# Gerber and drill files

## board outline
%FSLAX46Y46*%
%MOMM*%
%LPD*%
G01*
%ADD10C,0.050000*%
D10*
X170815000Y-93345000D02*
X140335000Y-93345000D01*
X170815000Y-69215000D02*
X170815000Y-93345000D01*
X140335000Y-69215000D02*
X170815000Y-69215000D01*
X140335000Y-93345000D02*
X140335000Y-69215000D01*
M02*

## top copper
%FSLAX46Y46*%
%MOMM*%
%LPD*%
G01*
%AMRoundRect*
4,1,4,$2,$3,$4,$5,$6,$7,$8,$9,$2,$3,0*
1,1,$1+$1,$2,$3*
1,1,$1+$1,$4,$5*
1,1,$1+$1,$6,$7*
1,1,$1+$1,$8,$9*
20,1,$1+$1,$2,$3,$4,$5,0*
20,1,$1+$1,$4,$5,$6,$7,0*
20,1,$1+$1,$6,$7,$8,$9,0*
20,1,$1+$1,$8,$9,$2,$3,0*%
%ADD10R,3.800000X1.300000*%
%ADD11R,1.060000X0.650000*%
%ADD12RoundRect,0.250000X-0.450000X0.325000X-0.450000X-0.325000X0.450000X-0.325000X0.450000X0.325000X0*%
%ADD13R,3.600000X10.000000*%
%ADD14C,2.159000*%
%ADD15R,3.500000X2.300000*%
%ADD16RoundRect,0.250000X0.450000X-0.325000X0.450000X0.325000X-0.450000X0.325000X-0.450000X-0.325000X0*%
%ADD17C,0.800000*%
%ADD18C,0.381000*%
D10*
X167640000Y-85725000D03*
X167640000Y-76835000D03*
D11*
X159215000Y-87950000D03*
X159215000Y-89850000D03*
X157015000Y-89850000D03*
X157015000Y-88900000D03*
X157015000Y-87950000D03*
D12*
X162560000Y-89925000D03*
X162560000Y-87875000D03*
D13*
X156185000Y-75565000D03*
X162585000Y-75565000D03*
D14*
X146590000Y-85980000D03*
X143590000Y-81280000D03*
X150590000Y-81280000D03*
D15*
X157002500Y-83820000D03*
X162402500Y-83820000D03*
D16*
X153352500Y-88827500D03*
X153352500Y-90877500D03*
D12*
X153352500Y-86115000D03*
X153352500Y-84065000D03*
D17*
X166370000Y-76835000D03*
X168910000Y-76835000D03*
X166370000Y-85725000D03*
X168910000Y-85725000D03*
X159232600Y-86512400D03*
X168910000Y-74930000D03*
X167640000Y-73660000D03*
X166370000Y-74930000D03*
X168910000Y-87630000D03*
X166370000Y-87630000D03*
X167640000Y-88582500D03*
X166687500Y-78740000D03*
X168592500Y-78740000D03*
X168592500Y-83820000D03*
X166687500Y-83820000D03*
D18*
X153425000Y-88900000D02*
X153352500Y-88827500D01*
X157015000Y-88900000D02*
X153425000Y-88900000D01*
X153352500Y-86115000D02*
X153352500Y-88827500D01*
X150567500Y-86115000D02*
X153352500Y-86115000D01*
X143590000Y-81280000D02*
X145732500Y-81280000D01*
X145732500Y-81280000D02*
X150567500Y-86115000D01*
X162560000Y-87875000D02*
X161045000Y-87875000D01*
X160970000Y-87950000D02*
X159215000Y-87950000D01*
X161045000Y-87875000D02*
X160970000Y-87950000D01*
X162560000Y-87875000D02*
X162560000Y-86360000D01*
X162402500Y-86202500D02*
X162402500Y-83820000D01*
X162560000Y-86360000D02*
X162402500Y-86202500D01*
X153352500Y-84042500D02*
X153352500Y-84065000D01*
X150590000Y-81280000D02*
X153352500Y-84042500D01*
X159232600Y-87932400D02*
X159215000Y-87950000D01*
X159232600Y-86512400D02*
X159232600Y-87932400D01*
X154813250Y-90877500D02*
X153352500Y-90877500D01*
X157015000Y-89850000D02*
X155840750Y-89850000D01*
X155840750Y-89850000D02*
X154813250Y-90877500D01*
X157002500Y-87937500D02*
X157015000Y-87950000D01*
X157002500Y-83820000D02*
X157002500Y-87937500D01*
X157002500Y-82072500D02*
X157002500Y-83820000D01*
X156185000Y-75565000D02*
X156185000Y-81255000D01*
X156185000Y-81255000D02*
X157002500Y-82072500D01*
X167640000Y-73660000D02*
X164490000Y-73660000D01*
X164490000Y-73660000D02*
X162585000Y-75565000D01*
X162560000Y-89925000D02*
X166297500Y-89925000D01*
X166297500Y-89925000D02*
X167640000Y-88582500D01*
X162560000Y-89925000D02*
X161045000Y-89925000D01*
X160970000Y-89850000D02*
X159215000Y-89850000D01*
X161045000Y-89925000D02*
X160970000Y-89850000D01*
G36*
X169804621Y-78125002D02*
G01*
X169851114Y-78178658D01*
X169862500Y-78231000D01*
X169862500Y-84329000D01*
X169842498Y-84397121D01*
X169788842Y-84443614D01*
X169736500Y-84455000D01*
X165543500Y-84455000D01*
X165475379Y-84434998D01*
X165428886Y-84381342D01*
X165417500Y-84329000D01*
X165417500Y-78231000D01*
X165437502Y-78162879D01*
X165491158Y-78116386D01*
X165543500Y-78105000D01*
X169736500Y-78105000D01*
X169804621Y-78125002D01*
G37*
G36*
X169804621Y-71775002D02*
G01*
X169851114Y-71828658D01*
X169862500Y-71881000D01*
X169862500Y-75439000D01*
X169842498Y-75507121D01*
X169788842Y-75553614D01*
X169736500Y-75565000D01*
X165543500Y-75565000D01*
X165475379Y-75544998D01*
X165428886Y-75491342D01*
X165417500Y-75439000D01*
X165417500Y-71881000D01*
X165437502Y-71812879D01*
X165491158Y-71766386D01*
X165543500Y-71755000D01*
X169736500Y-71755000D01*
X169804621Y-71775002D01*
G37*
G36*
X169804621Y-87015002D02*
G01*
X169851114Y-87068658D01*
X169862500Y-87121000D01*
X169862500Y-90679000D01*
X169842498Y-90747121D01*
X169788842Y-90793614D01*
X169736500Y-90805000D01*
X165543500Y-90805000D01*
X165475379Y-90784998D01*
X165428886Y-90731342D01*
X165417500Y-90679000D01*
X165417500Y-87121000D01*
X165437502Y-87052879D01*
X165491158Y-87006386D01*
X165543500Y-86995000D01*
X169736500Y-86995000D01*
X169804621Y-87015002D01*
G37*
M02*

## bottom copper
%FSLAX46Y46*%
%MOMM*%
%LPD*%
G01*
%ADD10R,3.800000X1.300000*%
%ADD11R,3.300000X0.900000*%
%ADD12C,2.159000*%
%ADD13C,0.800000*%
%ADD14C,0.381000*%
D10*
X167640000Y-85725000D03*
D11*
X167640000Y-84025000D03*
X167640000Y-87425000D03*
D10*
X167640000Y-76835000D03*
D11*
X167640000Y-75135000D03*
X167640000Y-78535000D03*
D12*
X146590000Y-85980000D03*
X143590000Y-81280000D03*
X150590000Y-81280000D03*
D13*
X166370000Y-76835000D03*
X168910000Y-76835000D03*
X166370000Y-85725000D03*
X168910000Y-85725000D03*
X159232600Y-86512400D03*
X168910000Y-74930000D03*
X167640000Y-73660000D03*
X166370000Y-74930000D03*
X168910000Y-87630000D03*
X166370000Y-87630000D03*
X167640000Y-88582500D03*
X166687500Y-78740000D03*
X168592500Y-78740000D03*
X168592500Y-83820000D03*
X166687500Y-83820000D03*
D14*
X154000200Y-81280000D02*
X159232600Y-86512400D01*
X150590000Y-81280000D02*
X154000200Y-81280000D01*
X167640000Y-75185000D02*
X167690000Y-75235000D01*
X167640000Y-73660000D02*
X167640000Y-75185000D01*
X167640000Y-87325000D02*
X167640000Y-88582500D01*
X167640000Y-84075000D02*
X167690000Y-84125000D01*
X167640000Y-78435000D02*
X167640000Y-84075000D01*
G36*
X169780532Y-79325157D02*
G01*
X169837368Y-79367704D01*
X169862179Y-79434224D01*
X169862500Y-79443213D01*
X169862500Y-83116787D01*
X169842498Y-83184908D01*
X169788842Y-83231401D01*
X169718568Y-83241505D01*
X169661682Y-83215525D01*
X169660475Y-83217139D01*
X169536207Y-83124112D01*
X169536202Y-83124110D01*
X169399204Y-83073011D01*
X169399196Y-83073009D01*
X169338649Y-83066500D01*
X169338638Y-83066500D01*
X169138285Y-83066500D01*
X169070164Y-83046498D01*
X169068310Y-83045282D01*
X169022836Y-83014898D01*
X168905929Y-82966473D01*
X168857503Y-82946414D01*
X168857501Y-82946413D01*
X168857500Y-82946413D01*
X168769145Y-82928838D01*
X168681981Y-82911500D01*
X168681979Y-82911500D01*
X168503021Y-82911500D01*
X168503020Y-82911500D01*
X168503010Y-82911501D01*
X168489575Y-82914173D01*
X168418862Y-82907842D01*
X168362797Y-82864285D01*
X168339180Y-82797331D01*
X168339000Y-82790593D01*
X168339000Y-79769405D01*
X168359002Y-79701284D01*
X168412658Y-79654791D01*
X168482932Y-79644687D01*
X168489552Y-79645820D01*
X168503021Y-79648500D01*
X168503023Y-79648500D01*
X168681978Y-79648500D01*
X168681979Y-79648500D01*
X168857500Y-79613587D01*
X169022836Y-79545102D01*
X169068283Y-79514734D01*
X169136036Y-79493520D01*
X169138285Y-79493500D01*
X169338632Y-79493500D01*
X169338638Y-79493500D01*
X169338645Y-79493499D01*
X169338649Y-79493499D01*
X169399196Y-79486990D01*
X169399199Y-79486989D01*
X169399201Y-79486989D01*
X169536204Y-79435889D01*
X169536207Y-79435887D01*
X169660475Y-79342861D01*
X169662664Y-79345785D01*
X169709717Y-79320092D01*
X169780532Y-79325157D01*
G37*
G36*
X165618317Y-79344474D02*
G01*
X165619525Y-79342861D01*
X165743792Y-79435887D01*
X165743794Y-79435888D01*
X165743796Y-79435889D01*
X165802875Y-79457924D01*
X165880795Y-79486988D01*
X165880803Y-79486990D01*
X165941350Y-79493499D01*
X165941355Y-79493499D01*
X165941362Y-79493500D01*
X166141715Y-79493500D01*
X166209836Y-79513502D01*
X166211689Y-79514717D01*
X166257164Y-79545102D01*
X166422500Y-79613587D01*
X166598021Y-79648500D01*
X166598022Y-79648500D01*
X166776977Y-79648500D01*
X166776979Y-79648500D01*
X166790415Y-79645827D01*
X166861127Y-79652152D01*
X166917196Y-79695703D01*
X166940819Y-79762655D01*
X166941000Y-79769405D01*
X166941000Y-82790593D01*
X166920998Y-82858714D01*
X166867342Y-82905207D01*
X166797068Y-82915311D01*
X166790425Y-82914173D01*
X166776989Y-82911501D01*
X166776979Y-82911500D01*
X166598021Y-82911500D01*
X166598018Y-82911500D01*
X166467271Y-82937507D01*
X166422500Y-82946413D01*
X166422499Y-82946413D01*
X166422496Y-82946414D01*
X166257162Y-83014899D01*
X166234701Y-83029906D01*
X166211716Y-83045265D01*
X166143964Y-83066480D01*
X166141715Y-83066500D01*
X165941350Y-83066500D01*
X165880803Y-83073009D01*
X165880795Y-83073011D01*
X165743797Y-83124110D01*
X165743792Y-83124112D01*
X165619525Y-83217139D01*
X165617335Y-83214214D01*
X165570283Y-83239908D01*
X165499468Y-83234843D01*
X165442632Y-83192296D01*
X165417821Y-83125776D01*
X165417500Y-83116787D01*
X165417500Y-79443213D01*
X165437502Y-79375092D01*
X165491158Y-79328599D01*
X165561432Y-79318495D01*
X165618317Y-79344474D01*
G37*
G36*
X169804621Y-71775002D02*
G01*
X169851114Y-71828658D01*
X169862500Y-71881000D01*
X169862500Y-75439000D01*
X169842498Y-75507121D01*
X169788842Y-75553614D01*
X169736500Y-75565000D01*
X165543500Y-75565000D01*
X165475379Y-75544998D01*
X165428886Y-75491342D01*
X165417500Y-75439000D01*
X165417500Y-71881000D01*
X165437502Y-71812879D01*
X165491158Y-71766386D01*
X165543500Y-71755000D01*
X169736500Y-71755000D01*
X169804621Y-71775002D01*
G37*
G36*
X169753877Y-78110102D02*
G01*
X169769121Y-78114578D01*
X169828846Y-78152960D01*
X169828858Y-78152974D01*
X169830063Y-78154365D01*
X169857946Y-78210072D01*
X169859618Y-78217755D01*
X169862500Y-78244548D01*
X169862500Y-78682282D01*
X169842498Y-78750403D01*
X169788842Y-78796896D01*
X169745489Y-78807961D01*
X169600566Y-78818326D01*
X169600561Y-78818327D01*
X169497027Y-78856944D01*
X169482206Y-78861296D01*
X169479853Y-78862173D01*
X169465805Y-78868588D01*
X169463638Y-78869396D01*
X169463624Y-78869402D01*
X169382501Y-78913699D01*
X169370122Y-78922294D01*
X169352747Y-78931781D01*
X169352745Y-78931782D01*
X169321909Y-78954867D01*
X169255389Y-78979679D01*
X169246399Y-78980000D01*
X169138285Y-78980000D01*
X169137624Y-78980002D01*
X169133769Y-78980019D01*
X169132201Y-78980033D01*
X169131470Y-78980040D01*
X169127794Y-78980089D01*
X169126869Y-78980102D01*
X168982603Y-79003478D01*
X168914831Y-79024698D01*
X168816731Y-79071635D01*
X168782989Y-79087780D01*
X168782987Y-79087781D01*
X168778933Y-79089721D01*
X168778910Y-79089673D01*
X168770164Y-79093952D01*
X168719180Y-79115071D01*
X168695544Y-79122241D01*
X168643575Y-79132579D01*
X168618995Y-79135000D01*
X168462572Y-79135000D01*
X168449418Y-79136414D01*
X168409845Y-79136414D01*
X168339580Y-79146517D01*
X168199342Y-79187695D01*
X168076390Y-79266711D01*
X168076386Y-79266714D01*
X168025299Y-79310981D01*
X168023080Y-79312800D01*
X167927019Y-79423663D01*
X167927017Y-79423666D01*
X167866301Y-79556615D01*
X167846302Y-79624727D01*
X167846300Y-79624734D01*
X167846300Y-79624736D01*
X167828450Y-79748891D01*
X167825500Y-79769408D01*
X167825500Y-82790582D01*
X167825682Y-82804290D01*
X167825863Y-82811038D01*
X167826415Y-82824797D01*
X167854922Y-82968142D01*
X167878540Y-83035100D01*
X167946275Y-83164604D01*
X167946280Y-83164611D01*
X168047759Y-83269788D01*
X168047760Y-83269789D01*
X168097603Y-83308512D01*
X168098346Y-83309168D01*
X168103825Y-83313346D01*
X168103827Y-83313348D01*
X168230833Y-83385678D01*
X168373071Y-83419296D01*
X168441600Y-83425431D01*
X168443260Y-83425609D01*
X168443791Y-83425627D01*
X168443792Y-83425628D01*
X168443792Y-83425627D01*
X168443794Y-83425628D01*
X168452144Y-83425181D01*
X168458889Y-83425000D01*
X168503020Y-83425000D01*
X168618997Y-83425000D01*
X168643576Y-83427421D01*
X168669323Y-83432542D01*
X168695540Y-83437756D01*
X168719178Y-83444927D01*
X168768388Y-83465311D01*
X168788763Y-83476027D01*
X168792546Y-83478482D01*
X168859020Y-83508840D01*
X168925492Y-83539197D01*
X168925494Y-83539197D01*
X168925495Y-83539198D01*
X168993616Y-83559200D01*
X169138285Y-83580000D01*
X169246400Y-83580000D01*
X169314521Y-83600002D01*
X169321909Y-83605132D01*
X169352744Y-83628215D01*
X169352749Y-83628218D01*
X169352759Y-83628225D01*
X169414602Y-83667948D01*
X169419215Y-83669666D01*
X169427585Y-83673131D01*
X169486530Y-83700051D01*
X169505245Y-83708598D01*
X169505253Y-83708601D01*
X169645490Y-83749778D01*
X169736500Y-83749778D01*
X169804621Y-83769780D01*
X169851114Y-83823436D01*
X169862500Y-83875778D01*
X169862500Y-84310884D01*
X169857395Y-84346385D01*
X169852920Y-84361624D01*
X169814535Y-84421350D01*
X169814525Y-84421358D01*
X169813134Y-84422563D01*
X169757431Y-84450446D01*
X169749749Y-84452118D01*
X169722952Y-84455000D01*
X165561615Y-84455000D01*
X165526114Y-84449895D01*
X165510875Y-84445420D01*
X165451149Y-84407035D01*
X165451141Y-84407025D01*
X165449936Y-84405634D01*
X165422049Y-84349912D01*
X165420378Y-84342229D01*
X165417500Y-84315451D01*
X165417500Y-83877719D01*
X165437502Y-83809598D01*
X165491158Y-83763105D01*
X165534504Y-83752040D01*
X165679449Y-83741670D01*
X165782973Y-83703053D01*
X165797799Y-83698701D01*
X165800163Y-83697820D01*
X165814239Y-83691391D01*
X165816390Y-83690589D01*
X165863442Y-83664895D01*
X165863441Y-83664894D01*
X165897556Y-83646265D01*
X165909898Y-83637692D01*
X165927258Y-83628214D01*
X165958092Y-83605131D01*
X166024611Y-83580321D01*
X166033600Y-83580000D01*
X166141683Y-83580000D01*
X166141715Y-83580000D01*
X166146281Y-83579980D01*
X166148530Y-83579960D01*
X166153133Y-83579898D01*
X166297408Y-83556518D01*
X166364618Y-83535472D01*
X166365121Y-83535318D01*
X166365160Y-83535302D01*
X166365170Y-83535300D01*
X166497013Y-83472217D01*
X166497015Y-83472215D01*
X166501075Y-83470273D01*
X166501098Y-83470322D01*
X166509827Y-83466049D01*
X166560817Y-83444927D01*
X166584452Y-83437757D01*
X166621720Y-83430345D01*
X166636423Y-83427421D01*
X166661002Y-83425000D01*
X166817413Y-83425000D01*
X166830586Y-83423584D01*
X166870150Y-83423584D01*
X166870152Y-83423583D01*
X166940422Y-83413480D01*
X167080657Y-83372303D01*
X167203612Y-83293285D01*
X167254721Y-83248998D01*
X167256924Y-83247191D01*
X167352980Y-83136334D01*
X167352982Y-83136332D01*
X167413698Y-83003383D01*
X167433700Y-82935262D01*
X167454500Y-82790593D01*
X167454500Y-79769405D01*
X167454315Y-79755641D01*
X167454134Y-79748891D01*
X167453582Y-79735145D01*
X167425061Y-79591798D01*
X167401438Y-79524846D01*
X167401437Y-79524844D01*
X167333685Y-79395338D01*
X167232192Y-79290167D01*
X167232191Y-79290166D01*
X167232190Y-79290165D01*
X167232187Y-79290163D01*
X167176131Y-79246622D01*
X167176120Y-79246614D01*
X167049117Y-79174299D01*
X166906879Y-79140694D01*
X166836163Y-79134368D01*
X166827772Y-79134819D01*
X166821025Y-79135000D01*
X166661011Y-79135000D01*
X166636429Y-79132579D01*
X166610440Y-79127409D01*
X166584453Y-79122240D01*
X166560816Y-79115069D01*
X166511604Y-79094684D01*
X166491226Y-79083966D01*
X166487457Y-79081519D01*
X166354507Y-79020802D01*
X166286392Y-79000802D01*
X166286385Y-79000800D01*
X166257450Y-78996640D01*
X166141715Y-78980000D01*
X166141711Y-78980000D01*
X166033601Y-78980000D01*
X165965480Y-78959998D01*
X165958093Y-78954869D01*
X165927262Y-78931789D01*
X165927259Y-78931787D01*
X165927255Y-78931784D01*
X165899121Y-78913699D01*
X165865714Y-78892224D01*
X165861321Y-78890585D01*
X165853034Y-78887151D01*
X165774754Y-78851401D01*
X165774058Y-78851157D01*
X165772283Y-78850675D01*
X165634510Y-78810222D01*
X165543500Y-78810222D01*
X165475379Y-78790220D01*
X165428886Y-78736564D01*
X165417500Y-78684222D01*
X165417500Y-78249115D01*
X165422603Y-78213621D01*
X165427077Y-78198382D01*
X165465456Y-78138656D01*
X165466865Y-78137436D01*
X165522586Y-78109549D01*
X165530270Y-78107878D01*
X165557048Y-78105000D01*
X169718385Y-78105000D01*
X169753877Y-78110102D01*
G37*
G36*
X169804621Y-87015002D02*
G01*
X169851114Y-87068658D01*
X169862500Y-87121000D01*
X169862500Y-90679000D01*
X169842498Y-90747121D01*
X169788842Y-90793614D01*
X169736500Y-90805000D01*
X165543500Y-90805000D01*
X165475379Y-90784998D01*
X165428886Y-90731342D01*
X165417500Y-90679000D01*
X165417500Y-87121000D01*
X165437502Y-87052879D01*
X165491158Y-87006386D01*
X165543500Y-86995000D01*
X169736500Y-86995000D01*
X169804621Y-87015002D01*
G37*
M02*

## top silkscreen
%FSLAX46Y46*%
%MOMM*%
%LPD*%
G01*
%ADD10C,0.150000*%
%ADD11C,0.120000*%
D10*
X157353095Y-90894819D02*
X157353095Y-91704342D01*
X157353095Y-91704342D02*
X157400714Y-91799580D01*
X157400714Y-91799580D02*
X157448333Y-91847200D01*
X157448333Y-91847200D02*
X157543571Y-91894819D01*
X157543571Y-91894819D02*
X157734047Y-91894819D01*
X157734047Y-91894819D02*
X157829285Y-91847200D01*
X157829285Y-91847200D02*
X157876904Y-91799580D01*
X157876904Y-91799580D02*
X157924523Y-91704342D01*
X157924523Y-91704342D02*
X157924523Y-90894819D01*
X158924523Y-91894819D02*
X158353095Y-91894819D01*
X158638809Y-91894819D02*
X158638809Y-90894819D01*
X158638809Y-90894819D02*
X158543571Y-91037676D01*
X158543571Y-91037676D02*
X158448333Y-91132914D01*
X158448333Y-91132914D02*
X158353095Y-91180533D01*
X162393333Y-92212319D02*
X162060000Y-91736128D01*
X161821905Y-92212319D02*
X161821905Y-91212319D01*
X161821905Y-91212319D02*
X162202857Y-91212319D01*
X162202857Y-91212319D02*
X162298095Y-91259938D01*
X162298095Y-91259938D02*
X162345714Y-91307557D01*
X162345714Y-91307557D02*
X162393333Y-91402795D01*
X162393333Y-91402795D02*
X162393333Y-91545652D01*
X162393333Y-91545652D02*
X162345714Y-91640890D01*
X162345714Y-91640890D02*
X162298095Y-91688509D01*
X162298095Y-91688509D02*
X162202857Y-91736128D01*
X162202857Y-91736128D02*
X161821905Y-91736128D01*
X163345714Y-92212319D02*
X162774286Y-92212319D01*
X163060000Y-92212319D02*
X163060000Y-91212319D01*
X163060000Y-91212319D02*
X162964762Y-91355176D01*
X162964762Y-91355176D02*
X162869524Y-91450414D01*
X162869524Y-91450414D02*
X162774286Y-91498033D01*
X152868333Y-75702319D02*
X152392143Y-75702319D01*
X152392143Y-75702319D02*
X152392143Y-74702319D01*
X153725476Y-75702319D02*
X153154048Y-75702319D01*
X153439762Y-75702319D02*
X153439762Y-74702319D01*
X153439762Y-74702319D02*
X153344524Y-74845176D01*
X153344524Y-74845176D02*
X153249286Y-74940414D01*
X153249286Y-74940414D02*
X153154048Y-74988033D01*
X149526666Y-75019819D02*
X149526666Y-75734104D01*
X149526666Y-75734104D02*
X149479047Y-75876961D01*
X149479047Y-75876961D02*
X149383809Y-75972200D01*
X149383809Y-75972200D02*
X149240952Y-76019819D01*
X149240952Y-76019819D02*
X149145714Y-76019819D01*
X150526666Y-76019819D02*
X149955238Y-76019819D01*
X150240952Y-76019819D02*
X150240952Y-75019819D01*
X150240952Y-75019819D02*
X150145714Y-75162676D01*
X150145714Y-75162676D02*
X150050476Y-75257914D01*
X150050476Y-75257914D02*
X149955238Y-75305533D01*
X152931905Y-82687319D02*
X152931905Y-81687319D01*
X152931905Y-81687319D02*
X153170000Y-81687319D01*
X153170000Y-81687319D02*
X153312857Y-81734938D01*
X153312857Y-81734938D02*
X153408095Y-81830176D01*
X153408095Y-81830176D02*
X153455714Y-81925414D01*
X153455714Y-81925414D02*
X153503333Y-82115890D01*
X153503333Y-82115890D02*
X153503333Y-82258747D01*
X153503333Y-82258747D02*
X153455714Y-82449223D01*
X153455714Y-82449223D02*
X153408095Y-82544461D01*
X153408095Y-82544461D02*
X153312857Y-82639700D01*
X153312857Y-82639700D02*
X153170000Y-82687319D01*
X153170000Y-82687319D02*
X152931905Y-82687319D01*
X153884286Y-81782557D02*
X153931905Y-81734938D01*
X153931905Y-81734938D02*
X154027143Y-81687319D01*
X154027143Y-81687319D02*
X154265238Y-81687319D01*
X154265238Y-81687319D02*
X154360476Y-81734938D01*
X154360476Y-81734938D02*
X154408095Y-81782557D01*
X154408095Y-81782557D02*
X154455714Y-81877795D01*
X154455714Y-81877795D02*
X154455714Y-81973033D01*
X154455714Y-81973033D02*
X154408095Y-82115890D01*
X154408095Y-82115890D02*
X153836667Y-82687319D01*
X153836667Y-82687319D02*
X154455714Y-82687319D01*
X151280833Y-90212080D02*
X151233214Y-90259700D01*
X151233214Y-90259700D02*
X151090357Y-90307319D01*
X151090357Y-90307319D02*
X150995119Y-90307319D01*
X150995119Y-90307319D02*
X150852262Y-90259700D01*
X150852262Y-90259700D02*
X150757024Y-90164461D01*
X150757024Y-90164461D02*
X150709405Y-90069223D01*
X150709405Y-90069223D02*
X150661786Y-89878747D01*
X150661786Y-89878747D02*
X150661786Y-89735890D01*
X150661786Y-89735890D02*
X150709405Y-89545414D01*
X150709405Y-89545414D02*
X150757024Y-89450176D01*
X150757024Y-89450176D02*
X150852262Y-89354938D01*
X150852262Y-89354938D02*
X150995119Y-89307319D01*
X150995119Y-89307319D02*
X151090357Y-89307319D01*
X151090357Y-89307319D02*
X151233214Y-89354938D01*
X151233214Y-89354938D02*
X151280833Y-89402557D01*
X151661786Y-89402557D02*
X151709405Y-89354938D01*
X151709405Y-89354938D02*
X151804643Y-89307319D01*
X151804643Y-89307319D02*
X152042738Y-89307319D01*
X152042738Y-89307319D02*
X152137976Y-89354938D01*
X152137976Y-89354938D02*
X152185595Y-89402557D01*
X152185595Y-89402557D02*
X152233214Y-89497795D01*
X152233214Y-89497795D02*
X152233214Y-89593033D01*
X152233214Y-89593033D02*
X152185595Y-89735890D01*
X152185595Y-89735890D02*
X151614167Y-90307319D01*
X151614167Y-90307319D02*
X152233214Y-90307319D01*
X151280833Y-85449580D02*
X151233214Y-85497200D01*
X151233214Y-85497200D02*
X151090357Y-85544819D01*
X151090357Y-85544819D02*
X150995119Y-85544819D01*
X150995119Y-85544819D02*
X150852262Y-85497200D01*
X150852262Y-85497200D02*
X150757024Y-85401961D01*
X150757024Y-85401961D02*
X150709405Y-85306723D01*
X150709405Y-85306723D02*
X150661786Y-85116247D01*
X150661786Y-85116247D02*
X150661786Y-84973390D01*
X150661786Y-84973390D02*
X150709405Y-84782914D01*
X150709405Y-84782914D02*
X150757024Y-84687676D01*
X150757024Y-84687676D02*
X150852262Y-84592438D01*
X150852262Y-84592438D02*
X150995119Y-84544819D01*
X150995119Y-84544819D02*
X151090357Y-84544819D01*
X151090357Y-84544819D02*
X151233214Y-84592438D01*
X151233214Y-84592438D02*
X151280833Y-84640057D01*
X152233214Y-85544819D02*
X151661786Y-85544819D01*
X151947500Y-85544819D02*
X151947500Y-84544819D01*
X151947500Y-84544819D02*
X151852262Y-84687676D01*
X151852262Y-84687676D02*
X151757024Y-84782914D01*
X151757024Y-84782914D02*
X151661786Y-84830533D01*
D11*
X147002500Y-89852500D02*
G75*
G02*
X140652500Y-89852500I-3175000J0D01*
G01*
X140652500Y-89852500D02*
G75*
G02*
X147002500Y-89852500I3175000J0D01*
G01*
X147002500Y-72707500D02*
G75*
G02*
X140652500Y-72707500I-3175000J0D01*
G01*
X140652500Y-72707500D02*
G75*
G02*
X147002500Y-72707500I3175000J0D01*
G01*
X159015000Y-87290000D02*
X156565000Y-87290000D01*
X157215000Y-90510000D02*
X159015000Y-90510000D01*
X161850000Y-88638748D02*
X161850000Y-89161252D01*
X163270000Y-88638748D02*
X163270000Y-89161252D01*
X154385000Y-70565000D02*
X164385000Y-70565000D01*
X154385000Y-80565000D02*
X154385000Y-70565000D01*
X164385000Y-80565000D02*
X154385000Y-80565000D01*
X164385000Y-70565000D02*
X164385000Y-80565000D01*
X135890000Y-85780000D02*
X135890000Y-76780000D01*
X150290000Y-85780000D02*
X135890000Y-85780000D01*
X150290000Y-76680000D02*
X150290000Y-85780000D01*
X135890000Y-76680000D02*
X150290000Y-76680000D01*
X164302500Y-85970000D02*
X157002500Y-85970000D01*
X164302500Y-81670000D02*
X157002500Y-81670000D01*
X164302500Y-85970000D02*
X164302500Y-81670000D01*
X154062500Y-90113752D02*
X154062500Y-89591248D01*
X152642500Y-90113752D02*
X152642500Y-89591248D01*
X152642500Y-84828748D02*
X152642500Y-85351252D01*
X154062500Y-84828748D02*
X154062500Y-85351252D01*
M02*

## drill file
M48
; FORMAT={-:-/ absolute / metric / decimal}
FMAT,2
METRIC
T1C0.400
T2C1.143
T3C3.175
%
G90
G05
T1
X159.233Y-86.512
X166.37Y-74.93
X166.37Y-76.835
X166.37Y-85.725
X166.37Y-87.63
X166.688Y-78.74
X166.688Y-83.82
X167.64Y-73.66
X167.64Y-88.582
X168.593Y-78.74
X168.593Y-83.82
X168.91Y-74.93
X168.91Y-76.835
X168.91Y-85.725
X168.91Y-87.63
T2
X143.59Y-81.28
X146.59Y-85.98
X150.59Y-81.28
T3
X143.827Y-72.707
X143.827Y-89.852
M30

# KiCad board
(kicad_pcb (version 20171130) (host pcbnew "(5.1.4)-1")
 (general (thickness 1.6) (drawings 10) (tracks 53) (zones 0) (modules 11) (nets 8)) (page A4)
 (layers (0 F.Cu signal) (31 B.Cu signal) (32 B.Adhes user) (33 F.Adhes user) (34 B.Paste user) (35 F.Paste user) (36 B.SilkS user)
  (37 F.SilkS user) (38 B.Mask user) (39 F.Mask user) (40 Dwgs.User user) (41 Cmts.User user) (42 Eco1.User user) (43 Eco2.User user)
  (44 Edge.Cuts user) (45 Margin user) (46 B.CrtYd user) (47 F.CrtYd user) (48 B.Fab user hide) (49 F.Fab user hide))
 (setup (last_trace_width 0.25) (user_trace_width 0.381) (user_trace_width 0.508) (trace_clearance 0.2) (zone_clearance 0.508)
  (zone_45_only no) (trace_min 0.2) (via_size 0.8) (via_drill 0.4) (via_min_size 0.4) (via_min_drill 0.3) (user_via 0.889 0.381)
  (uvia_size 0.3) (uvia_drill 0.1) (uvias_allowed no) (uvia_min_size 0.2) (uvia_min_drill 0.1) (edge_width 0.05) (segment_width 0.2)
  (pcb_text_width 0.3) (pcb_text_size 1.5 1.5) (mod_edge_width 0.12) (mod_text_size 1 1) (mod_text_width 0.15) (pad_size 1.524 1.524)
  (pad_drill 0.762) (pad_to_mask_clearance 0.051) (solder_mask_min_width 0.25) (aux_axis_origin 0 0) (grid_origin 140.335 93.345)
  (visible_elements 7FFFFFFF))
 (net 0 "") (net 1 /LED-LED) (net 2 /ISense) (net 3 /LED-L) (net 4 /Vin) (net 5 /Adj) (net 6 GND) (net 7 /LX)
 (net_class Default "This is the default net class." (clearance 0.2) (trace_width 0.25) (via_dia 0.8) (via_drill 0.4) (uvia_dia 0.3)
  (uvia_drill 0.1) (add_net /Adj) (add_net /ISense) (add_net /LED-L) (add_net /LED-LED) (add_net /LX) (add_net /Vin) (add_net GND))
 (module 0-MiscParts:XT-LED (layer B.Cu) (at 167.64 85.725 90)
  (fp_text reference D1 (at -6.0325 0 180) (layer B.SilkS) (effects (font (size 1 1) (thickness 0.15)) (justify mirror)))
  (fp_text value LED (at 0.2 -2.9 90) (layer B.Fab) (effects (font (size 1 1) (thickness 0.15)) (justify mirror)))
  (pad "" smd rect (at 0 0 90) (size 1.3 3.8) (layers F.Cu B.Paste B.Mask))
  (pad "" smd rect (at 0 0 90) (size 1.3 3.8) (layers B.Cu B.Paste B.Mask))
  (pad 1 smd rect (at 1.7 0 90) (size 0.9 3.3) (layers B.Cu B.Paste B.Mask) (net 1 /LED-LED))
  (pad 2 smd rect (at -1.7 0 90) (size 0.9 3.3) (layers B.Cu B.Paste B.Mask) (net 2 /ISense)))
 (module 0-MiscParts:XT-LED (layer B.Cu) (at 167.64 76.835 90)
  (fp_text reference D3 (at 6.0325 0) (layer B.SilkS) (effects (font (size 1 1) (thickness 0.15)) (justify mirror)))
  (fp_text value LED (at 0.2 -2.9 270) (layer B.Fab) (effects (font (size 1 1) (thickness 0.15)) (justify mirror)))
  (pad "" smd rect (at 0 0 90) (size 1.3 3.8) (layers F.Cu B.Paste B.Mask))
  (pad "" smd rect (at 0 0 90) (size 1.3 3.8) (layers B.Cu B.Paste B.Mask))
  (pad 1 smd rect (at 1.7 0 90) (size 0.9 3.3) (layers B.Cu B.Paste B.Mask) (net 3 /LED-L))
  (pad 2 smd rect (at -1.7 0 90) (size 0.9 3.3) (layers B.Cu B.Paste B.Mask) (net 1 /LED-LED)))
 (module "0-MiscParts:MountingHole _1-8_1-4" (layer F.Cu) (at 143.8275 89.8525)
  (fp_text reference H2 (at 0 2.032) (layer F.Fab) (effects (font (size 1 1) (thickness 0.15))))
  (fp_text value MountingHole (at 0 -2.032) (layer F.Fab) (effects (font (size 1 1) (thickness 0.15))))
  (fp_circle (center 0 0) (end 3.175 0) (layer F.SilkS) (width 0.12))
  (pad "" np_thru_hole circle (at 0 0) (size 3.175 3.175) (drill 3.175) (layers *.Cu *.Mask)))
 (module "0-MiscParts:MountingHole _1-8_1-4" (layer F.Cu) (at 143.8275 72.7075)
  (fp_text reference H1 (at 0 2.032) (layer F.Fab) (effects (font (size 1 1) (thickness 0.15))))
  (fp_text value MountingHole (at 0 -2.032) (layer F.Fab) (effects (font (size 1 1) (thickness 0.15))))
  (fp_circle (center 0 0) (end 3.175 0) (layer F.SilkS) (width 0.12))
  (pad "" np_thru_hole circle (at 0 0) (size 3.175 3.175) (drill 3.175) (layers *.Cu *.Mask)))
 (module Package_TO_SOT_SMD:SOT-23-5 (layer F.Cu) (at 158.115 88.9)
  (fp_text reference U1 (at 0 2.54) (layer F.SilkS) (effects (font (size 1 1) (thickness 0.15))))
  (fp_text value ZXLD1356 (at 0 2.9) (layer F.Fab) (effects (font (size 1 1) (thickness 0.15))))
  (fp_line (start 0.9 -1.61) (end -1.55 -1.61) (layer F.SilkS) (width 0.12))
  (fp_line (start -0.9 1.61) (end 0.9 1.61) (layer F.SilkS) (width 0.12))
  (pad 5 smd rect (at 1.1 -0.95) (size 1.06 0.65) (layers F.Cu F.Paste F.Mask) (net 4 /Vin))
  (pad 4 smd rect (at 1.1 0.95) (size 1.06 0.65) (layers F.Cu F.Paste F.Mask) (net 2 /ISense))
  (pad 3 smd rect (at -1.1 0.95) (size 1.06 0.65) (layers F.Cu F.Paste F.Mask) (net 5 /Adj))
  (pad 2 smd rect (at -1.1 0) (size 1.06 0.65) (layers F.Cu F.Paste F.Mask) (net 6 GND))
  (pad 1 smd rect (at -1.1 -0.95) (size 1.06 0.65) (layers F.Cu F.Paste F.Mask) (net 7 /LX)))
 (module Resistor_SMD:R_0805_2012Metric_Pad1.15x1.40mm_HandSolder (layer F.Cu) (at 162.56 88.9 270)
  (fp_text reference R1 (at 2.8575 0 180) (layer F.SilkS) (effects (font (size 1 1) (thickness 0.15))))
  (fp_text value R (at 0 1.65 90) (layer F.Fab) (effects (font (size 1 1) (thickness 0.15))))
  (fp_line (start -0.261252 0.71) (end 0.261252 0.71) (layer F.SilkS) (width 0.12))
  (fp_line (start -0.261252 -0.71) (end 0.261252 -0.71) (layer F.SilkS) (width 0.12))
  (pad 2 smd roundrect (at 1.025 0 270) (size 1.15 1.4) (layers F.Cu F.Paste F.Mask) (roundrect_rratio 0.217391) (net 2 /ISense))
  (pad 1 smd roundrect (at -1.025 0 270) (size 1.15 1.4) (layers F.Cu F.Paste F.Mask) (roundrect_rratio 0.217391) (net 4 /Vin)))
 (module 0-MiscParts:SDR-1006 (layer F.Cu) (at 159.385 75.565 270)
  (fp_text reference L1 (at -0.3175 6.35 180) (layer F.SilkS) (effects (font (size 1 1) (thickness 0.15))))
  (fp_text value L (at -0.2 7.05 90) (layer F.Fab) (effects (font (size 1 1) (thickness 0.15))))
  (fp_line (start -5 5) (end -5 -5) (layer F.SilkS) (width 0.12))
  (fp_line (start 5 5) (end -5 5) (layer F.SilkS) (width 0.12))
  (fp_line (start 5 -5) (end 5 5) (layer F.SilkS) (width 0.12))
  (fp_line (start -5 -5) (end 5 -5) (layer F.SilkS) (width 0.12))
  (pad 2 smd rect (at 0 3.2 270) (size 10 3.6) (layers F.Cu F.Paste F.Mask) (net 7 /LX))
  (pad 1 smd rect (at 0 -3.2 270) (size 10 3.6) (layers F.Cu F.Paste F.Mask) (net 3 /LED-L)))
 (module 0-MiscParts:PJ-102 (layer F.Cu) (at 135.89 81.28)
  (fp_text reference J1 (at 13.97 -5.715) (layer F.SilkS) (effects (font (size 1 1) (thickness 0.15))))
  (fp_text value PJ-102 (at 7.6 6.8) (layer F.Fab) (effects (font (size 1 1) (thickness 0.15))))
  (fp_line (start 0 4.5) (end 0 -4.5) (layer F.SilkS) (width 0.12))
  (fp_line (start 14.4 4.5) (end 0 4.5) (layer F.SilkS) (width 0.12))
  (fp_line (start 14.4 -4.6) (end 14.4 4.5) (layer F.SilkS) (width 0.12))
  (fp_line (start 0 -4.6) (end 14.4 -4.6) (layer F.SilkS) (width 0.12))
  (pad 3 thru_hole circle (at 10.7 4.7) (size 2.159 2.159) (drill 1.143) (layers *.Cu *.Mask))
  (pad 2 thru_hole circle (at 7.7 0) (size 2.159 2.159) (drill 1.143) (layers *.Cu *.Mask) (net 6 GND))
  (pad 1 thru_hole circle (at 14.7 0) (size 2.159 2.159) (drill 1.143) (layers *.Cu *.Mask) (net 4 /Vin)))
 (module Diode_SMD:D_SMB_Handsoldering (layer F.Cu) (at 159.7025 83.82 180)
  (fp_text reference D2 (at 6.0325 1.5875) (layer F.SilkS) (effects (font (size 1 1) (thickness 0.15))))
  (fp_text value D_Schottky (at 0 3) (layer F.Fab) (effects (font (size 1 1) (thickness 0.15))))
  (fp_line (start -4.6 -2.15) (end 2.7 -2.15) (layer F.SilkS) (width 0.12))
  (fp_line (start -4.6 2.15) (end 2.7 2.15) (layer F.SilkS) (width 0.12))
  (fp_line (start -4.6 -2.15) (end -4.6 2.15) (layer F.SilkS) (width 0.12))
  (pad 2 smd rect (at 2.7 0 180) (size 3.5 2.3) (layers F.Cu F.Paste F.Mask) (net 7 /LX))
  (pad 1 smd rect (at -2.7 0 180) (size 3.5 2.3) (layers F.Cu F.Paste F.Mask) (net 4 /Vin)))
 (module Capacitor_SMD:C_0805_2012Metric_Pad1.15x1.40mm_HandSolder (layer F.Cu) (at 153.3525 89.8525 90)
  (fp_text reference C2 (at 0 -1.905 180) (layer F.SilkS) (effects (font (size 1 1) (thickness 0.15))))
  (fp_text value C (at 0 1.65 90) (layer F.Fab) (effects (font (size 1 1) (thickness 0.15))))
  (fp_line (start -0.261252 0.71) (end 0.261252 0.71) (layer F.SilkS) (width 0.12))
  (fp_line (start -0.261252 -0.71) (end 0.261252 -0.71) (layer F.SilkS) (width 0.12))
  (pad 2 smd roundrect (at 1.025 0 90) (size 1.15 1.4) (layers F.Cu F.Paste F.Mask) (roundrect_rratio 0.217391) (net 6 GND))
  (pad 1 smd roundrect (at -1.025 0 90) (size 1.15 1.4) (layers F.Cu F.Paste F.Mask) (roundrect_rratio 0.217391) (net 5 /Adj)))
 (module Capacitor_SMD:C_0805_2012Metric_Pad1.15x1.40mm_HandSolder (layer F.Cu) (at 153.3525 85.09 270)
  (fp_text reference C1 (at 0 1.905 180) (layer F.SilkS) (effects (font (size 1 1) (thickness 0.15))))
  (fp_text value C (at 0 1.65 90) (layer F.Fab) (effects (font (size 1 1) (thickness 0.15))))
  (fp_line (start -0.261252 0.71) (end 0.261252 0.71) (layer F.SilkS) (width 0.12))
  (fp_line (start -0.261252 -0.71) (end 0.261252 -0.71) (layer F.SilkS) (width 0.12))
  (pad 2 smd roundrect (at 1.025 0 270) (size 1.15 1.4) (layers F.Cu F.Paste F.Mask) (roundrect_rratio 0.217391) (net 6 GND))
  (pad 1 smd roundrect (at -1.025 0 270) (size 1.15 1.4) (layers F.Cu F.Paste F.Mask) (roundrect_rratio 0.217391) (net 4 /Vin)))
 (gr_line (start 170.815 93.345) (end 140.335 93.345) (layer Edge.Cuts) (width 0.05))
 (gr_line (start 170.815 69.215) (end 170.815 93.345) (layer Edge.Cuts) (width 0.05))
 (gr_line (start 140.335 69.215) (end 170.815 69.215) (layer Edge.Cuts) (width 0.05))
 (gr_line (start 140.335 93.345) (end 140.335 69.215) (layer Edge.Cuts) (width 0.05))
 (via (at 166.37 76.835) (size 0.8) (drill 0.4) (layers F.Cu B.Cu) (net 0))
 (via (at 168.91 76.835) (size 0.8) (drill 0.4) (layers F.Cu B.Cu) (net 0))
 (via (at 166.37 85.725) (size 0.8) (drill 0.4) (layers F.Cu B.Cu) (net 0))
 (via (at 168.91 85.725) (size 0.8) (drill 0.4) (layers F.Cu B.Cu) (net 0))
 (segment (start 153.425 88.9) (end 153.3525 88.8275) (width 0.381) (layer F.Cu) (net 6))
 (segment (start 157.015 88.9) (end 153.425 88.9) (width 0.381) (layer F.Cu) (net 6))
 (segment (start 153.3525 86.115) (end 153.3525 88.8275) (width 0.381) (layer F.Cu) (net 6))
 (segment (start 150.5675 86.115) (end 153.3525 86.115) (width 0.381) (layer F.Cu) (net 6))
 (segment (start 143.59 81.28) (end 145.7325 81.28) (width 0.381) (layer F.Cu) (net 6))
 (segment (start 145.7325 81.28) (end 150.5675 86.115) (width 0.381) (layer F.Cu) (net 6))
 (via (at 159.2326 86.5124) (size 0.8) (drill 0.4) (layers F.Cu B.Cu) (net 4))
 (segment (start 162.56 87.875) (end 161.045 87.875) (width 0.381) (layer F.Cu) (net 4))
 (segment (start 160.97 87.95) (end 159.215 87.95) (width 0.381) (layer F.Cu) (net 4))
 (segment (start 161.045 87.875) (end 160.97 87.95) (width 0.381) (layer F.Cu) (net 4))
 (segment (start 162.56 87.875) (end 162.56 86.36) (width 0.381) (layer F.Cu) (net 4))
 (segment (start 162.4025 86.2025) (end 162.4025 83.82) (width 0.381) (layer F.Cu) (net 4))
 (segment (start 162.56 86.36) (end 162.4025 86.2025) (width 0.381) (layer F.Cu) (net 4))
 (segment (start 154.0002 81.28) (end 159.2326 86.5124) (width 0.381) (layer B.Cu) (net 4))
 (segment (start 150.59 81.28) (end 154.0002 81.28) (width 0.381) (layer B.Cu) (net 4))
 (segment (start 153.3525 84.0425) (end 153.3525 84.065) (width 0.381) (layer F.Cu) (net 4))
 (segment (start 150.59 81.28) (end 153.3525 84.0425) (width 0.381) (layer F.Cu) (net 4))
 (segment (start 159.2326 87.9324) (end 159.215 87.95) (width 0.381) (layer F.Cu) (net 4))
 (segment (start 159.2326 86.5124) (end 159.2326 87.9324) (width 0.381) (layer F.Cu) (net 4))
 (segment (start 154.81325 90.8775) (end 153.3525 90.8775) (width 0.381) (layer F.Cu) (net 5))
 (segment (start 157.015 89.85) (end 155.84075 89.85) (width 0.381) (layer F.Cu) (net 5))
 (segment (start 155.84075 89.85) (end 154.81325 90.8775) (width 0.381) (layer F.Cu) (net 5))
 (segment (start 157.0025 87.9375) (end 157.015 87.95) (width 0.381) (layer F.Cu) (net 7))
 (segment (start 157.0025 83.82) (end 157.0025 87.9375) (width 0.381) (layer F.Cu) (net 7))
 (segment (start 157.0025 82.0725) (end 157.0025 83.82) (width 0.381) (layer F.Cu) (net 7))
 (segment (start 156.185 75.565) (end 156.185 81.255) (width 0.381) (layer F.Cu) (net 7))
 (segment (start 156.185 81.255) (end 157.0025 82.0725) (width 0.381) (layer F.Cu) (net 7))
 (via (at 168.91 74.93) (size 0.8) (drill 0.4) (layers F.Cu B.Cu) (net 3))
 (segment (start 167.64 75.185) (end 167.69 75.235) (width 0.381) (layer B.Cu) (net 3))
 (via (at 167.64 73.66) (size 0.8) (drill 0.4) (layers F.Cu B.Cu) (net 3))
 (segment (start 167.64 73.66) (end 164.49 73.66) (width 0.381) (layer F.Cu) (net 3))
 (segment (start 164.49 73.66) (end 162.585 75.565) (width 0.381) (layer F.Cu) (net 3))
 (segment (start 167.64 73.66) (end 167.64 75.185) (width 0.381) (layer B.Cu) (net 3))
 (via (at 166.37 74.93) (size 0.8) (drill 0.4) (layers F.Cu B.Cu) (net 3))
 (via (at 168.91 87.63) (size 0.8) (drill 0.4) (layers F.Cu B.Cu) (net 2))
 (via (at 166.37 87.63) (size 0.8) (drill 0.4) (layers F.Cu B.Cu) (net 2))
 (via (at 167.64 88.5825) (size 0.8) (drill 0.4) (layers F.Cu B.Cu) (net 2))
 (segment (start 162.56 89.925) (end 166.2975 89.925) (width 0.381) (layer F.Cu) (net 2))
 (segment (start 166.2975 89.925) (end 167.64 88.5825) (width 0.381) (layer F.Cu) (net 2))
 (segment (start 167.64 87.325) (end 167.64 88.5825) (width 0.381) (layer B.Cu) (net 2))
 (segment (start 162.56 89.925) (end 161.045 89.925) (width 0.381) (layer F.Cu) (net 2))
 (segment (start 160.97 89.85) (end 159.215 89.85) (width 0.381) (layer F.Cu) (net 2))
 (segment (start 161.045 89.925) (end 160.97 89.85) (width 0.381) (layer F.Cu) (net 2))
 (via (at 166.6875 78.74) (size 0.8) (drill 0.4) (layers F.Cu B.Cu) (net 1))
 (via (at 168.5925 78.74) (size 0.8) (drill 0.4) (layers F.Cu B.Cu) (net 1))
 (via (at 168.5925 83.82) (size 0.8) (drill 0.4) (layers F.Cu B.Cu) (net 1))
 (via (at 166.6875 83.82) (size 0.8) (drill 0.4) (layers F.Cu B.Cu) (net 1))
 (segment (start 167.64 84.075) (end 167.69 84.125) (width 0.381) (layer B.Cu) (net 1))
 (segment (start 167.64 78.435) (end 167.64 84.075) (width 0.381) (layer B.Cu) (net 1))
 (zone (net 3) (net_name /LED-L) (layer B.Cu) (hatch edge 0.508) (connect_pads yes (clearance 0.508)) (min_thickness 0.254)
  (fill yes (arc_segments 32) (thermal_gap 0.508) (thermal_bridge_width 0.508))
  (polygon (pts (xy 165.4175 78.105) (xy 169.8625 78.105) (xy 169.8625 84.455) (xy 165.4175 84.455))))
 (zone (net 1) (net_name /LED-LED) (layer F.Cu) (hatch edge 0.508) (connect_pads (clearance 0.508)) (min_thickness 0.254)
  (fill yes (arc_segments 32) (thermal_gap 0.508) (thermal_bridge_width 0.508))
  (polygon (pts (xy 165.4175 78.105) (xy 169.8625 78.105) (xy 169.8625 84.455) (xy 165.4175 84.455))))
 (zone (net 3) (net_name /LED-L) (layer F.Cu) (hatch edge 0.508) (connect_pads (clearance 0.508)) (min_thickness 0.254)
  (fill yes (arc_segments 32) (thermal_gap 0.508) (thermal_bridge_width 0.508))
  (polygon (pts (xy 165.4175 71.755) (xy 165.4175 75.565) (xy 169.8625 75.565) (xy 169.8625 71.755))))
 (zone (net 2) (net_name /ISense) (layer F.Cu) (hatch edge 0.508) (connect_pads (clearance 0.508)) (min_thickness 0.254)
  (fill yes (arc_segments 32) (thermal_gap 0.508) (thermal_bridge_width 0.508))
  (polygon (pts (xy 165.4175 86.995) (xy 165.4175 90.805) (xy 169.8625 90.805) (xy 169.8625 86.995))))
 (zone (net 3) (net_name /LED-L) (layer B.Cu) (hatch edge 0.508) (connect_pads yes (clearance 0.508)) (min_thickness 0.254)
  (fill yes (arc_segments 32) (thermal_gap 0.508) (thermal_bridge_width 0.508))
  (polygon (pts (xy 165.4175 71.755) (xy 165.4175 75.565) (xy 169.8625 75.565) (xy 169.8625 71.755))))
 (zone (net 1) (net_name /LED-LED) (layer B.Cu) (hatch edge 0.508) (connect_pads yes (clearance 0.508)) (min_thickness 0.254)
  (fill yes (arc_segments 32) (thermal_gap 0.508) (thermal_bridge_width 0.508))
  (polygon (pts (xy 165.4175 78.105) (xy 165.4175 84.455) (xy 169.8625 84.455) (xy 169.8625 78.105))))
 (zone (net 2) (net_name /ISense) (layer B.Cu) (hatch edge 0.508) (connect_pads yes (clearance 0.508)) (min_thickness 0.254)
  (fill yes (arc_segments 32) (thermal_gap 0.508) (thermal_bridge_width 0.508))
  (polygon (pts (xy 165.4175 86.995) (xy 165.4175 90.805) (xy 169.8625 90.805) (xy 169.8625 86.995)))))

